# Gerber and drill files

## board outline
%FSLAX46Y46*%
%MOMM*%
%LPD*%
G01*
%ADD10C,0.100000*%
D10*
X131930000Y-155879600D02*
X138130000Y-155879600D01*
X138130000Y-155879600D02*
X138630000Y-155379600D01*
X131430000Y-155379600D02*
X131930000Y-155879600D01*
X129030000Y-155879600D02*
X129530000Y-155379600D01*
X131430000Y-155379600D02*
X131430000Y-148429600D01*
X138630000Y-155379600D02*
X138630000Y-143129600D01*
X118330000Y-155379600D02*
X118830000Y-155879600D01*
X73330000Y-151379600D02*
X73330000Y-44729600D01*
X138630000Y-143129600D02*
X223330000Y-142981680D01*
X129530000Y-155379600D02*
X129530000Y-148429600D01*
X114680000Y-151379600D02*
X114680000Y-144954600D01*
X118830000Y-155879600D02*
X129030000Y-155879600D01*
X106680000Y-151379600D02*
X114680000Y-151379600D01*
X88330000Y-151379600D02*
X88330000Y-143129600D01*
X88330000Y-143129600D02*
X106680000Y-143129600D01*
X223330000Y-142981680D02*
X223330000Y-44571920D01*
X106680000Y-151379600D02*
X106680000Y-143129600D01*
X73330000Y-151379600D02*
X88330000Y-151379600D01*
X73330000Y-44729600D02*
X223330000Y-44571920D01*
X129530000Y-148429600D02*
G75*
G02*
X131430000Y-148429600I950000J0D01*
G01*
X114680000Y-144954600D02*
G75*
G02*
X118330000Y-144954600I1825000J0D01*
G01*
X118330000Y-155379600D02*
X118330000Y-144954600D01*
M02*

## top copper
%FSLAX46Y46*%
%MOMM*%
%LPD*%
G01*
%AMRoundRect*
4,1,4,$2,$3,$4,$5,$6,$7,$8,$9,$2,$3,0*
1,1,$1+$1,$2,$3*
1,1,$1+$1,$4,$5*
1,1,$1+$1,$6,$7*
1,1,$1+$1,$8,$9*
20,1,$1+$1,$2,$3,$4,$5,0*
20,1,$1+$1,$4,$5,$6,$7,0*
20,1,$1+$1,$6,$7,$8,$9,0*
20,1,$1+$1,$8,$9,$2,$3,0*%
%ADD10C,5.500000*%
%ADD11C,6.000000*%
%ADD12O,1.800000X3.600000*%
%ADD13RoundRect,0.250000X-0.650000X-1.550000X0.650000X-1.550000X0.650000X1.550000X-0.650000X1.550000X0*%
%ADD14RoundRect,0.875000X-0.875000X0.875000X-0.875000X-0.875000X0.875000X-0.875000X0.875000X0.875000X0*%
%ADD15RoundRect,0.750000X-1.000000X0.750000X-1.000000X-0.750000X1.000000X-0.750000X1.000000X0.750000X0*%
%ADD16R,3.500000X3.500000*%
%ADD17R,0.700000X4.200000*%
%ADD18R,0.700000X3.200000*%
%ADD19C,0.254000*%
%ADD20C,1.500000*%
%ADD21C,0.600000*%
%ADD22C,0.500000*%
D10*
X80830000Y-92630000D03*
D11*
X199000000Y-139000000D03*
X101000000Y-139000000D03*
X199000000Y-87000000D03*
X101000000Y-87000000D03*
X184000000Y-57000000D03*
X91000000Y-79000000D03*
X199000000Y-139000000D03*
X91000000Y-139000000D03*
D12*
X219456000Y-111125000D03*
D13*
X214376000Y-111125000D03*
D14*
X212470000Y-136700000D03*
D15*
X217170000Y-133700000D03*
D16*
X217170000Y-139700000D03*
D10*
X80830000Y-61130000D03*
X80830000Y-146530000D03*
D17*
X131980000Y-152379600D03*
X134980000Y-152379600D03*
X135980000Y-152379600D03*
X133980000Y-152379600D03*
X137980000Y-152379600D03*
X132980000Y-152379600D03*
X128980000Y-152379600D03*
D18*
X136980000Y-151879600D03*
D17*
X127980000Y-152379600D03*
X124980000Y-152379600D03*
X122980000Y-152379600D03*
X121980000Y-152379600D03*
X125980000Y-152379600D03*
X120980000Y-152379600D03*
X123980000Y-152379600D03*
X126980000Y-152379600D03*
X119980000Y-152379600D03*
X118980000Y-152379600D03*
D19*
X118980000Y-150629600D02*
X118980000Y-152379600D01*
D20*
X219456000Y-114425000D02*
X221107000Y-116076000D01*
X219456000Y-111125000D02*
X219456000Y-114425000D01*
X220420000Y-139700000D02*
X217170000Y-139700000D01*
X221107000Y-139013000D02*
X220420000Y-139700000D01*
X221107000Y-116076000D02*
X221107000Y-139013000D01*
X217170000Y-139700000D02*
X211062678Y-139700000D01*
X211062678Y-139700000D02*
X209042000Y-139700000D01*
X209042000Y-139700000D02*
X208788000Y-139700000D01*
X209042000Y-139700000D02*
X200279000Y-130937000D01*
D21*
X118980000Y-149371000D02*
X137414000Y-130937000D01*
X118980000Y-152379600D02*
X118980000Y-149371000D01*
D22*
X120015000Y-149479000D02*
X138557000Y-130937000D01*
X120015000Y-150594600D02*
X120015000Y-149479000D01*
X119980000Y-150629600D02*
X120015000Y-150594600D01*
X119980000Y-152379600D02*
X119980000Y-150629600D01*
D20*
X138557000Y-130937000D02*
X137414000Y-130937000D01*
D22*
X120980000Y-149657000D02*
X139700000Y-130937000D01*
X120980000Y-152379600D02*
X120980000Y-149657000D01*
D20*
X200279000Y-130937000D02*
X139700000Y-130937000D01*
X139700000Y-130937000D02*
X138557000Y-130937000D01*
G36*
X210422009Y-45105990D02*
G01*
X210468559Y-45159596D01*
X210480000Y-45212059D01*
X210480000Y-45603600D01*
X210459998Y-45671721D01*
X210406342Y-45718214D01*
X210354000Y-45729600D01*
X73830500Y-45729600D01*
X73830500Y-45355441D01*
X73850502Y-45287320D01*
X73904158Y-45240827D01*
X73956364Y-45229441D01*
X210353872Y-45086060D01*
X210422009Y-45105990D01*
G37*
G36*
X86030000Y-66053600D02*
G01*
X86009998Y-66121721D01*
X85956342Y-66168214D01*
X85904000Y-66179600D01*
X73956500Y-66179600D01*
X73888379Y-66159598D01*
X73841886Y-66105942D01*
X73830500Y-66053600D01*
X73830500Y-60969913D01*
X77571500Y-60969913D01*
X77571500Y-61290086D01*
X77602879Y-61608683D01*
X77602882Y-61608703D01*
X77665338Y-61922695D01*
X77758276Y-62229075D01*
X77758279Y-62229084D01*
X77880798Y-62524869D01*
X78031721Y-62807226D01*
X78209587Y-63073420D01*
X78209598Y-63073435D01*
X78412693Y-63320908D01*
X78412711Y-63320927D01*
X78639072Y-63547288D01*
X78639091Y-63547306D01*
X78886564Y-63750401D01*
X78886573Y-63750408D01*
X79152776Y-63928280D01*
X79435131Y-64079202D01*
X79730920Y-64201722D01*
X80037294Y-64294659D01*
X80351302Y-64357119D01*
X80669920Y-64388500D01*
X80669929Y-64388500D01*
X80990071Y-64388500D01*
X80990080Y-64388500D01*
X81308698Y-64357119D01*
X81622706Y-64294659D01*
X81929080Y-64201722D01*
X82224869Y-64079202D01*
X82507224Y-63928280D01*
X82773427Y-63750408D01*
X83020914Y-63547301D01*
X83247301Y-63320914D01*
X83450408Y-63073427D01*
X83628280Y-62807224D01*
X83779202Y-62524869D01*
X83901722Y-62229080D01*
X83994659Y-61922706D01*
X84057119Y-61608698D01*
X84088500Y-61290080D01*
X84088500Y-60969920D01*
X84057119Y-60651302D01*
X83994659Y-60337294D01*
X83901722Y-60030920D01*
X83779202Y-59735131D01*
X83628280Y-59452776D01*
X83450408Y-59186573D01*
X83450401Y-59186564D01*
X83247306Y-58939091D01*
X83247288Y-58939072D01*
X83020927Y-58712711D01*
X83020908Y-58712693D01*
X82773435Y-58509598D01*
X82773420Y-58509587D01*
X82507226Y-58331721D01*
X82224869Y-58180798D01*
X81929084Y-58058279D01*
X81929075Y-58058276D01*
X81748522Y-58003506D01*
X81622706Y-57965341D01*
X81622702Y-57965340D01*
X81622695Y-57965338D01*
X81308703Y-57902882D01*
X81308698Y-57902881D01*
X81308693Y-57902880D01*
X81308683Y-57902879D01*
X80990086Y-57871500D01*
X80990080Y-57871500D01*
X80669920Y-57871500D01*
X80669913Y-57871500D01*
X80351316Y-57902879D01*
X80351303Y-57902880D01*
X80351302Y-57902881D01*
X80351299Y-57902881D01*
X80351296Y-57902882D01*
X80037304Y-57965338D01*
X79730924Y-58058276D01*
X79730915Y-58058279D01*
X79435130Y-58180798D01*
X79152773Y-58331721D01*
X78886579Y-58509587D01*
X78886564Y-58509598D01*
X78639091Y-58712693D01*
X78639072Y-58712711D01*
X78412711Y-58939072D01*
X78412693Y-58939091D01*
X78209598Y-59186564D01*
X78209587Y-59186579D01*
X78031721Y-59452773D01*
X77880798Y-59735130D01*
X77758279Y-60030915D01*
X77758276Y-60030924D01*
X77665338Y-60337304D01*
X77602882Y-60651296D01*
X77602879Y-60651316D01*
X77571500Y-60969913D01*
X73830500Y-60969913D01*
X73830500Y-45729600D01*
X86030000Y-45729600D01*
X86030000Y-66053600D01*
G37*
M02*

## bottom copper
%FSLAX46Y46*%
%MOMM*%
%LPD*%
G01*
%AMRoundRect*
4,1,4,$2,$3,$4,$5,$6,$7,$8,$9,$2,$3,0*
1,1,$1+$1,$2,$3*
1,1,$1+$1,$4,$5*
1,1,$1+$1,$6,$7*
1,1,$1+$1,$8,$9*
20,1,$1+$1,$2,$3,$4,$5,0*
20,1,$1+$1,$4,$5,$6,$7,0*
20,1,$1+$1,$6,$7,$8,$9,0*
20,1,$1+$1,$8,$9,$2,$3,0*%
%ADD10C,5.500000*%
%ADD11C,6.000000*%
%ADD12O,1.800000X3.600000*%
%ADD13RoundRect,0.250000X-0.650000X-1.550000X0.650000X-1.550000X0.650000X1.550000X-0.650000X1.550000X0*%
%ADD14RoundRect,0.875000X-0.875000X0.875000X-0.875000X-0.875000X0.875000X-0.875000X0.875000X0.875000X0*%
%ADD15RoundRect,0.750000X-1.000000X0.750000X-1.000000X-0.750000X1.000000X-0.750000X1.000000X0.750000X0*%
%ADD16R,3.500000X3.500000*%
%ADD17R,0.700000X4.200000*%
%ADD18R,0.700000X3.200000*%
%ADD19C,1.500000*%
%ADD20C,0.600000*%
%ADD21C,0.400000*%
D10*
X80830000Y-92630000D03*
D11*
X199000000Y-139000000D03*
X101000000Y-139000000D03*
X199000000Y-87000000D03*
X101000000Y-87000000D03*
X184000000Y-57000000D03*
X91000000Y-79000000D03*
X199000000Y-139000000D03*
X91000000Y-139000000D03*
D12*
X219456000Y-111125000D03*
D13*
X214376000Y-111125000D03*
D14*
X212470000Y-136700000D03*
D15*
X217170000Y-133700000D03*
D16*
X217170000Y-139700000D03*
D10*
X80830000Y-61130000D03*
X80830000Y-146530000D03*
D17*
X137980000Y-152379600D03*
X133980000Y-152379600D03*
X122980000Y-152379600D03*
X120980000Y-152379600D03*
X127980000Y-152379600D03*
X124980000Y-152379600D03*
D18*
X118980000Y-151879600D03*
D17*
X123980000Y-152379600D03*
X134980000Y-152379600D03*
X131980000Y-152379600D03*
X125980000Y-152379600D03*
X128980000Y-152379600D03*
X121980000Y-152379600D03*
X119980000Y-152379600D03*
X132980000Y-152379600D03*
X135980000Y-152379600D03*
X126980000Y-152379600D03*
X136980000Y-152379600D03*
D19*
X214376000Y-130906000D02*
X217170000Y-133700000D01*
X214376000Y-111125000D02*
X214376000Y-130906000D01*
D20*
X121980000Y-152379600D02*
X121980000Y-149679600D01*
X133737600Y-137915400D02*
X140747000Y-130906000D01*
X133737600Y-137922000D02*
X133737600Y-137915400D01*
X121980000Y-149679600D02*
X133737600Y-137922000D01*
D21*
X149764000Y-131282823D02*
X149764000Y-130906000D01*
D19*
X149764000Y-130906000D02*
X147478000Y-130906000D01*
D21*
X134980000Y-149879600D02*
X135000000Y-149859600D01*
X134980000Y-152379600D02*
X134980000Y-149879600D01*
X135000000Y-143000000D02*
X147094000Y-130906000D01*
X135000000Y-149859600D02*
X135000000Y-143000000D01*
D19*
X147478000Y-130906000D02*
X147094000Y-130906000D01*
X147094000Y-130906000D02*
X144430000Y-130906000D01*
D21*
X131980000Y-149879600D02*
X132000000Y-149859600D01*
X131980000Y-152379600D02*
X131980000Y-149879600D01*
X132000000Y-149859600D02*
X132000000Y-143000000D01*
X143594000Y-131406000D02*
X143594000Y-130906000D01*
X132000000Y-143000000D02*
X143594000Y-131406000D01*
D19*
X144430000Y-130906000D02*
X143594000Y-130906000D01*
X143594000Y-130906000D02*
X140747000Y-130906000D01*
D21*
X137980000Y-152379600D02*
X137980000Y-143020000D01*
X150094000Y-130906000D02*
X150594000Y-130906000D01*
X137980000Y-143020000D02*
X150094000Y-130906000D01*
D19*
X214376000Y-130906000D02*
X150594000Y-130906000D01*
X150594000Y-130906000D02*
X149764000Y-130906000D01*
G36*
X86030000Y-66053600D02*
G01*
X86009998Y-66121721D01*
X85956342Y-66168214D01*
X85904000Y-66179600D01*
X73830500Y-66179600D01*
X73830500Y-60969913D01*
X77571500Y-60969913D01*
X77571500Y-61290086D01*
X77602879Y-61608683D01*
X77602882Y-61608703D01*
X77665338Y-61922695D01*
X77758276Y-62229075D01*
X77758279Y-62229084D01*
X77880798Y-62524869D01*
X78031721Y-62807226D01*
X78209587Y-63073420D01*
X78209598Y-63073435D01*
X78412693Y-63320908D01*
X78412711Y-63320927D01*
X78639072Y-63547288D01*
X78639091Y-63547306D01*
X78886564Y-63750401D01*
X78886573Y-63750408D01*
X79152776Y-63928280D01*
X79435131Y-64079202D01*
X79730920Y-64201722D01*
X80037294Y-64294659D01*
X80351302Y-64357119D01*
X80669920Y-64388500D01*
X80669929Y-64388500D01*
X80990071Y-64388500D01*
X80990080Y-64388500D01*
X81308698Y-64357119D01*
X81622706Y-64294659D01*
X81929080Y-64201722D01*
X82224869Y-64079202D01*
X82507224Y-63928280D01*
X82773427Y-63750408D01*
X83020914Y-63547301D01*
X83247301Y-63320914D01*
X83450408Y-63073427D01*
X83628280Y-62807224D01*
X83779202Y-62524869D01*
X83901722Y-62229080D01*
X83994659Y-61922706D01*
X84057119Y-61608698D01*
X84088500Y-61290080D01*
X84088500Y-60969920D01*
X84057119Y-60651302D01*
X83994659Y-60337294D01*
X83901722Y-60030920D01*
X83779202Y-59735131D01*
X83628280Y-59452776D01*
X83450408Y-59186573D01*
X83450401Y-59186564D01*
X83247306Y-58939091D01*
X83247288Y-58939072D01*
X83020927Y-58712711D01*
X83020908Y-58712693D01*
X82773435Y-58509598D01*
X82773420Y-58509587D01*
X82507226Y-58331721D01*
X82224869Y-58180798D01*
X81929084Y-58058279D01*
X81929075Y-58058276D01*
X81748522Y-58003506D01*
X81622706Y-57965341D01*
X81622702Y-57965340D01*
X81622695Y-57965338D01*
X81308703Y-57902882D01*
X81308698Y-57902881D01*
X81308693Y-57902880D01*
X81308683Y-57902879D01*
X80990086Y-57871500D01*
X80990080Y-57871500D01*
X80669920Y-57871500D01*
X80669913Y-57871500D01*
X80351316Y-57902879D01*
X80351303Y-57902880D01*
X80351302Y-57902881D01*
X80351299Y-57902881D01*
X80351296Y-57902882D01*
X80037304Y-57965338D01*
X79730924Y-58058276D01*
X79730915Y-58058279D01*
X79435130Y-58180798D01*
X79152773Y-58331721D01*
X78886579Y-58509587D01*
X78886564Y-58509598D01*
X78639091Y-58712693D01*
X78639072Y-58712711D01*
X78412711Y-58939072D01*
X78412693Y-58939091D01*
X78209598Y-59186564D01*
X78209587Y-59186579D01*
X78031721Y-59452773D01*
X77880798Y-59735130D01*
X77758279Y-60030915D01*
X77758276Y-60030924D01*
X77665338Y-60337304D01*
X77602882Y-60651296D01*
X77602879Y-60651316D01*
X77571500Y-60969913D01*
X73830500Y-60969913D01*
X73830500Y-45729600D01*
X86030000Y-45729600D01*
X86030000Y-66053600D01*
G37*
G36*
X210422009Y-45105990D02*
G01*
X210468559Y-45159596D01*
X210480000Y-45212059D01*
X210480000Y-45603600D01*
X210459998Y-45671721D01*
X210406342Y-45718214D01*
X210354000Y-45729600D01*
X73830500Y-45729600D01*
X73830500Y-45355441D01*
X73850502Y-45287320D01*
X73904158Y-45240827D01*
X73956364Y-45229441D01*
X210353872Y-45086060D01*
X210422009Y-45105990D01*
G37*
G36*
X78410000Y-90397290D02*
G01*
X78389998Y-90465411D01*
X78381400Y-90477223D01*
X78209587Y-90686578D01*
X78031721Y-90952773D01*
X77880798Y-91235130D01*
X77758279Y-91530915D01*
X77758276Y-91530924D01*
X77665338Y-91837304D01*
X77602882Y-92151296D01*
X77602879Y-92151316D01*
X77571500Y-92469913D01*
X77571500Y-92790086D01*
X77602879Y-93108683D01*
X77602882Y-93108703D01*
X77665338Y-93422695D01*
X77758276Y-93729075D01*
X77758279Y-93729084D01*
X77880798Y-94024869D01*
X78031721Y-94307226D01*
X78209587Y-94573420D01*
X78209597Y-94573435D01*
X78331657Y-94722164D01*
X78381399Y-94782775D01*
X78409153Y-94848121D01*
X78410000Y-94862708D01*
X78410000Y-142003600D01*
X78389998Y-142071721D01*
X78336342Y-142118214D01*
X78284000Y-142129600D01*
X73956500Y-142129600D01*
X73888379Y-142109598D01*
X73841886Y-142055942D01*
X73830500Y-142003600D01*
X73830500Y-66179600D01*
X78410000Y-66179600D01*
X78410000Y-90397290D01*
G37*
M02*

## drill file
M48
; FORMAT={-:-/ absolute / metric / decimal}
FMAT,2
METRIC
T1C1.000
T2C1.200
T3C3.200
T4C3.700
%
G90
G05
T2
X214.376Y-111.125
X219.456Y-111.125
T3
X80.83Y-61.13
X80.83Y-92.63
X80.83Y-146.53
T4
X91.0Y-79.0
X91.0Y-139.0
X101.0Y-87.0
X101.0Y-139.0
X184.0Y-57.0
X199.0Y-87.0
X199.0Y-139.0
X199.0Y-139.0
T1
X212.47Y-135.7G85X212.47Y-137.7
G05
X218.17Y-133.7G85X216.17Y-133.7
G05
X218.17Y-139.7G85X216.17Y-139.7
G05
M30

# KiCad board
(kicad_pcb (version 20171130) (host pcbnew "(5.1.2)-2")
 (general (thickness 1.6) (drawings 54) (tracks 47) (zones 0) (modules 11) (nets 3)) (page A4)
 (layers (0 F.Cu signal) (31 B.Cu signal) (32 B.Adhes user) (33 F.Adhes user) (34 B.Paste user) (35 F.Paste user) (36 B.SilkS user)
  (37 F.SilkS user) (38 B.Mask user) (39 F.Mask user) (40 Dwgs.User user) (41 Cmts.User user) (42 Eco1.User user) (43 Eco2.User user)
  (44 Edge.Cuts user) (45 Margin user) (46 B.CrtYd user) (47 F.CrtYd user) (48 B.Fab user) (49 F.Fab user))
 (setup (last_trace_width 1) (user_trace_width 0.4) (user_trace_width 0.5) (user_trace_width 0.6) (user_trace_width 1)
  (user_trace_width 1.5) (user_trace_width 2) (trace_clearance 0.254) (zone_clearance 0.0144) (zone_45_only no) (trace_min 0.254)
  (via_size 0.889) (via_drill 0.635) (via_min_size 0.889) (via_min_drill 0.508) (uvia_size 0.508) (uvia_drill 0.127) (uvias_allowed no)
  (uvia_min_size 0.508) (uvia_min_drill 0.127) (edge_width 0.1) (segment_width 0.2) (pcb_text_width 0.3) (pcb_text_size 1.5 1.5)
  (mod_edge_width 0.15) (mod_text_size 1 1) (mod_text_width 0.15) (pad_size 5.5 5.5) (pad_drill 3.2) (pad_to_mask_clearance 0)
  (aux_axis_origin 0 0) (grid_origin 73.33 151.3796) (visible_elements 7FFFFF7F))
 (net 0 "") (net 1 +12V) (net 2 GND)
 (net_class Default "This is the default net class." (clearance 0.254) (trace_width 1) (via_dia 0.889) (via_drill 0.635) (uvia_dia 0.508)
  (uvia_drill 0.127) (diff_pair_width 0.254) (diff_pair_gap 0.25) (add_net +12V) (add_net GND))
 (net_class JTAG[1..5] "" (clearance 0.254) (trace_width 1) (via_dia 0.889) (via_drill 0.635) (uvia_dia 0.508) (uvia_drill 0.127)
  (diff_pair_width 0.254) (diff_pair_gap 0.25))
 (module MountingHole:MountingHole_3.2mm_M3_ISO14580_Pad (layer F.Cu) (at 80.83 92.63)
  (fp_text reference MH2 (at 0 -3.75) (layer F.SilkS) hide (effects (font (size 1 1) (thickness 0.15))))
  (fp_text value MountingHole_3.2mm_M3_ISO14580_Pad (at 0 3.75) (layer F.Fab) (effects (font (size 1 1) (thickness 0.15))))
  (pad 1 thru_hole circle (at 0 0) (size 5.5 5.5) (drill 3.2) (layers *.Cu *.Mask)))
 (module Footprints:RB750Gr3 (layer F.Cu) (at 150 113)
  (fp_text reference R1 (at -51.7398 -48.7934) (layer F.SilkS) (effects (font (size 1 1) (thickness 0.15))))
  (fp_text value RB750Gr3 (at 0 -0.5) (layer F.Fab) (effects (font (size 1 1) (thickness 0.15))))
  (pad 4 thru_hole circle (at 49 26) (size 6 6) (drill 3.7) (layers *.Cu *.Mask))
  (pad 3 thru_hole circle (at -49 26) (size 6 6) (drill 3.7) (layers *.Cu *.Mask))
  (pad 2 thru_hole circle (at 49 -26) (size 6 6) (drill 3.7) (layers *.Cu *.Mask))
  (pad 1 thru_hole circle (at -49 -26) (size 6 6) (drill 3.7) (layers *.Cu *.Mask)))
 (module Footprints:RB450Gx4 (layer F.Cu) (at 87 53)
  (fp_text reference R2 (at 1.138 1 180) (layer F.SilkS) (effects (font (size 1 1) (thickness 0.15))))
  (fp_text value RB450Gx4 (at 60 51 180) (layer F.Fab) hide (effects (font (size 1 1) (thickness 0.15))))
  (pad 2 thru_hole circle (at 97 4 180) (size 6 6) (drill 3.7) (layers *.Cu *.Mask))
  (pad 1 thru_hole circle (at 4 26 180) (size 6 6) (drill 3.7) (layers *.Cu *.Mask))
  (pad 4 thru_hole circle (at 112 86 180) (size 6 6) (drill 3.7) (layers *.Cu *.Mask))
  (pad 3 thru_hole circle (at 4 86 180) (size 6 6) (drill 3.7) (layers *.Cu *.Mask)))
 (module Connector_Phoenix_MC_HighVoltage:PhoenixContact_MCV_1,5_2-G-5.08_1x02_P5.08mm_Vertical (layer F.Cu) (at 214.376 111.125)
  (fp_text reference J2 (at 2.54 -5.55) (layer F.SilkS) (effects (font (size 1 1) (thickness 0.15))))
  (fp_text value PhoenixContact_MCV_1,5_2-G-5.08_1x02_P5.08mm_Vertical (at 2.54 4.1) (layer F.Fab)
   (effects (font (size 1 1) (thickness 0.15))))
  (pad 2 thru_hole oval (at 5.08 0) (size 1.8 3.6) (drill 1.2) (layers *.Cu *.Mask) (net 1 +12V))
  (pad 1 thru_hole roundrect (at 0 0) (size 1.8 3.6) (drill 1.2) (layers *.Cu *.Mask) (roundrect_rratio 0.138889) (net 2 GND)))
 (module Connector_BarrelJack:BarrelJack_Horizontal (layer F.Cu) (at 217.17 139.7 270)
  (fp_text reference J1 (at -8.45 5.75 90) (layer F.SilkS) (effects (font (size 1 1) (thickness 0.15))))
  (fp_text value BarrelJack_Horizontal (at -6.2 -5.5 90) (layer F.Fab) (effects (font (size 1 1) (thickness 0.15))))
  (pad 3 thru_hole roundrect (at -3 4.7 270) (size 3.5 3.5) (drill oval 3 1) (layers *.Cu *.Mask) (roundrect_rratio 0.25))
  (pad 2 thru_hole roundrect (at -6 0 270) (size 3 3.5) (drill oval 1 3) (layers *.Cu *.Mask) (roundrect_rratio 0.25) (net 2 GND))
  (pad 1 thru_hole rect (at 0 0 270) (size 3.5 3.5) (drill oval 1 3) (layers *.Cu *.Mask) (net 1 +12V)))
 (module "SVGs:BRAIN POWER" (layer B.Cu) (at 155.575 97.79 180)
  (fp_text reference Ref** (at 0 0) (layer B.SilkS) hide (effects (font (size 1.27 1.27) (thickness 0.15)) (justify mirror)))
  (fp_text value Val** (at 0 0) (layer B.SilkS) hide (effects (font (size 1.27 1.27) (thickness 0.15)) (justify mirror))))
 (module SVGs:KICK (layer F.Cu) (at 148.9456 53.4416)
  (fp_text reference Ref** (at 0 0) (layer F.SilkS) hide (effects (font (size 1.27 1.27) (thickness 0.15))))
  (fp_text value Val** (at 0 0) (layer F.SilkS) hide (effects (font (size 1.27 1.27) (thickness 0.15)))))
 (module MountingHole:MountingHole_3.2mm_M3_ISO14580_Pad (layer F.Cu) (at 80.83 61.13)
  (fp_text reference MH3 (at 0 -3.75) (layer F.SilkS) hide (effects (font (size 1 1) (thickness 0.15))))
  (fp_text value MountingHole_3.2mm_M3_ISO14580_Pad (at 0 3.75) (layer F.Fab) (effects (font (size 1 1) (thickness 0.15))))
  (pad 2 thru_hole circle (at 0 0) (size 5.5 5.5) (drill 3.2) (layers *.Cu *.Mask)))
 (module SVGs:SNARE (layer B.Cu) (at 148.1582 53.5178 180)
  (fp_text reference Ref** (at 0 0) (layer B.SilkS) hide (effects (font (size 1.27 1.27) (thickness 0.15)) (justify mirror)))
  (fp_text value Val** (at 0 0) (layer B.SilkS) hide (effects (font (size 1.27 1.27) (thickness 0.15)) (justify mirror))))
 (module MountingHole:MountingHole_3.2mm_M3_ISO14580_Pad (layer F.Cu) (at 80.83 146.53)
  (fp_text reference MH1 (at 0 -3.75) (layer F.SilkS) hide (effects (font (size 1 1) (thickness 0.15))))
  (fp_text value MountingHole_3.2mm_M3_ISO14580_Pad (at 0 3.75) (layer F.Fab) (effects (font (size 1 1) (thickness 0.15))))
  (pad 1 thru_hole circle (at 0 0) (size 5.5 5.5) (drill 3.2) (layers *.Cu *.Mask)))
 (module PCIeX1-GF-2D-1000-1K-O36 (layer F.Cu) (at 128.48 152.3796)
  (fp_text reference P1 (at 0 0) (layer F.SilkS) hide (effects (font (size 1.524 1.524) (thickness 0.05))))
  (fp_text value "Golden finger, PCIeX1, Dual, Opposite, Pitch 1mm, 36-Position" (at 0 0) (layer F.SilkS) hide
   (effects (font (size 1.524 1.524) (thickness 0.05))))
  (pad B12 smd rect (at 3.5 0) (size 0.7 4.2) (layers F.Cu F.Paste F.Mask))
  (pad B15 smd rect (at 6.5 0) (size 0.7 4.2) (layers F.Cu F.Paste F.Mask))
  (pad B16 smd rect (at 7.5 0) (size 0.7 4.2) (layers F.Cu F.Paste F.Mask))
  (pad B14 smd rect (at 5.5 0) (size 0.7 4.2) (layers F.Cu F.Paste F.Mask))
  (pad B18 smd rect (at 9.5 0) (size 0.7 4.2) (layers F.Cu F.Paste F.Mask))
  (pad B13 smd rect (at 4.5 0) (size 0.7 4.2) (layers F.Cu F.Paste F.Mask))
  (pad B11 smd rect (at 0.5 0) (size 0.7 4.2) (layers F.Cu F.Paste F.Mask))
  (pad B17 smd rect (at 8.5 -0.5) (size 0.7 3.2) (layers F.Cu F.Paste F.Mask))
  (pad B10 smd rect (at -0.5 0) (size 0.7 4.2) (layers F.Cu F.Paste F.Mask))
  (pad B7 smd rect (at -3.5 0) (size 0.7 4.2) (layers F.Cu F.Paste F.Mask))
  (pad B5 smd rect (at -5.5 0) (size 0.7 4.2) (layers F.Cu F.Paste F.Mask))
  (pad B4 smd rect (at -6.5 0) (size 0.7 4.2) (layers F.Cu F.Paste F.Mask))
  (pad B8 smd rect (at -2.5 0) (size 0.7 4.2) (layers F.Cu F.Paste F.Mask))
  (pad B3 smd rect (at -7.5 0) (size 0.7 4.2) (layers F.Cu F.Paste F.Mask) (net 1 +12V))
  (pad B6 smd rect (at -4.5 0) (size 0.7 4.2) (layers F.Cu F.Paste F.Mask))
  (pad B9 smd rect (at -1.5 0) (size 0.7 4.2) (layers F.Cu F.Paste F.Mask))
  (pad B2 smd rect (at -8.5 0) (size 0.7 4.2) (layers F.Cu F.Paste F.Mask) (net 1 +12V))
  (pad B1 smd rect (at -9.5 0) (size 0.7 4.2) (layers F.Cu F.Paste F.Mask) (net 1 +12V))
  (pad A18 smd rect (at 9.5 0) (size 0.7 4.2) (layers B.Cu B.Paste B.Mask) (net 2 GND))
  (pad A14 smd rect (at 5.5 0) (size 0.7 4.2) (layers B.Cu B.Paste B.Mask))
  (pad A5 smd rect (at -5.5 0) (size 0.7 4.2) (layers B.Cu B.Paste B.Mask))
  (pad A3 smd rect (at -7.5 0) (size 0.7 4.2) (layers B.Cu B.Paste B.Mask))
  (pad A10 smd rect (at -0.5 0) (size 0.7 4.2) (layers B.Cu B.Paste B.Mask))
  (pad A7 smd rect (at -3.5 0) (size 0.7 4.2) (layers B.Cu B.Paste B.Mask))
  (pad A1 smd rect (at -9.5 -0.5) (size 0.7 3.2) (layers B.Cu B.Paste B.Mask))
  (pad A6 smd rect (at -4.5 0) (size 0.7 4.2) (layers B.Cu B.Paste B.Mask))
  (pad A15 smd rect (at 6.5 0) (size 0.7 4.2) (layers B.Cu B.Paste B.Mask) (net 2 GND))
  (pad A12 smd rect (at 3.5 0) (size 0.7 4.2) (layers B.Cu B.Paste B.Mask) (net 2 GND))
  (pad A8 smd rect (at -2.5 0) (size 0.7 4.2) (layers B.Cu B.Paste B.Mask))
  (pad A11 smd rect (at 0.5 0) (size 0.7 4.2) (layers B.Cu B.Paste B.Mask))
  (pad A4 smd rect (at -6.5 0) (size 0.7 4.2) (layers B.Cu B.Paste B.Mask) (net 2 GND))
  (pad A2 smd rect (at -8.5 0) (size 0.7 4.2) (layers B.Cu B.Paste B.Mask))
  (pad A13 smd rect (at 4.5 0) (size 0.7 4.2) (layers B.Cu B.Paste B.Mask))
  (pad A16 smd rect (at 7.5 0) (size 0.7 4.2) (layers B.Cu B.Paste B.Mask))
  (pad A9 smd rect (at -1.5 0) (size 0.7 4.2) (layers B.Cu B.Paste B.Mask))
  (pad A17 smd rect (at 8.5 0) (size 0.7 4.2) (layers B.Cu B.Paste B.Mask)))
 (gr_line (start 131.93 155.8796) (end 138.13 155.8796) (layer Edge.Cuts) (width 0.1))
 (gr_line (start 138.13 155.8796) (end 138.63 155.3796) (layer Edge.Cuts) (width 0.1))
 (gr_line (start 131.43 155.3796) (end 131.93 155.8796) (layer Edge.Cuts) (width 0.1))
 (gr_line (start 129.03 155.8796) (end 129.53 155.3796) (layer Edge.Cuts) (width 0.1))
 (gr_line (start 131.43 155.3796) (end 131.43 148.4296) (layer Edge.Cuts) (width 0.1))
 (gr_line (start 138.63 155.3796) (end 138.63 143.1296) (layer Edge.Cuts) (width 0.1))
 (gr_line (start 118.33 155.3796) (end 118.83 155.8796) (layer Edge.Cuts) (width 0.1))
 (gr_line (start 73.33 151.3796) (end 73.33 44.7296) (layer Edge.Cuts) (width 0.1))
 (gr_line (start 138.63 143.1296) (end 223.33 142.98168) (layer Edge.Cuts) (width 0.1))
 (gr_line (start 129.53 155.3796) (end 129.53 148.4296) (layer Edge.Cuts) (width 0.1))
 (gr_line (start 114.68 151.3796) (end 114.68 144.9546) (layer Edge.Cuts) (width 0.1))
 (gr_line (start 118.83 155.8796) (end 129.03 155.8796) (layer Edge.Cuts) (width 0.1))
 (gr_line (start 106.68 151.3796) (end 114.68 151.3796) (layer Edge.Cuts) (width 0.1))
 (gr_line (start 88.33 151.3796) (end 88.33 143.1296) (layer Edge.Cuts) (width 0.1))
 (gr_line (start 88.33 143.1296) (end 106.68 143.1296) (layer Edge.Cuts) (width 0.1))
 (gr_line (start 223.33 142.98168) (end 223.33 44.57192) (layer Edge.Cuts) (width 0.1))
 (gr_line (start 106.68 151.3796) (end 106.68 143.1296) (layer Edge.Cuts) (width 0.1))
 (gr_line (start 73.33 151.3796) (end 88.33 151.3796) (layer Edge.Cuts) (width 0.1))
 (gr_line (start 73.33 44.7296) (end 223.33 44.57192) (layer Edge.Cuts) (width 0.1))
 (gr_arc (start 130.48 148.4296) (end 131.43 148.4296) (angle -180) (layer Edge.Cuts) (width 0.1))
 (gr_arc (start 116.505 144.9546) (end 118.33 144.9546) (angle -180) (layer Edge.Cuts) (width 0.1))
 (gr_line (start 118.33 155.3796) (end 118.33 144.9546) (layer Edge.Cuts) (width 0.1))
 (segment (start 214.376 130.906) (end 217.17 133.7) (width 1.5) (layer B.Cu) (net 2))
 (segment (start 214.376 111.125) (end 214.376 130.906) (width 1.5) (layer B.Cu) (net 2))
 (segment (start 121.98 152.3796) (end 121.98 149.6796) (width 0.6) (layer B.Cu) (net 2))
 (segment (start 133.7376 137.9154) (end 140.747 130.906) (width 0.6) (layer B.Cu) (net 2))
 (segment (start 133.7376 137.922) (end 133.7376 137.9154) (width 0.6) (layer B.Cu) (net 2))
 (segment (start 121.98 149.6796) (end 133.7376 137.922) (width 0.6) (layer B.Cu) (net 2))
 (segment (start 149.764 131.282823) (end 149.764 130.906) (width 0.4) (layer B.Cu) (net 2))
 (segment (start 149.764 130.906) (end 147.478 130.906) (width 1.5) (layer B.Cu) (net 2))
 (segment (start 134.98 149.8796) (end 135 149.8596) (width 0.4) (layer B.Cu) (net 2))
 (segment (start 134.98 152.3796) (end 134.98 149.8796) (width 0.4) (layer B.Cu) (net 2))
 (segment (start 135 143) (end 147.094 130.906) (width 0.4) (layer B.Cu) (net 2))
 (segment (start 135 149.8596) (end 135 143) (width 0.4) (layer B.Cu) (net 2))
 (segment (start 147.478 130.906) (end 147.094 130.906) (width 1.5) (layer B.Cu) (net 2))
 (segment (start 147.094 130.906) (end 144.43 130.906) (width 1.5) (layer B.Cu) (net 2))
 (segment (start 131.98 149.8796) (end 132 149.8596) (width 0.4) (layer B.Cu) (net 2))
 (segment (start 131.98 152.3796) (end 131.98 149.8796) (width 0.4) (layer B.Cu) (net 2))
 (segment (start 132 149.8596) (end 132 143) (width 0.4) (layer B.Cu) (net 2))
 (segment (start 143.594 131.406) (end 143.594 130.906) (width 0.4) (layer B.Cu) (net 2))
 (segment (start 132 143) (end 143.594 131.406) (width 0.4) (layer B.Cu) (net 2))
 (segment (start 144.43 130.906) (end 143.594 130.906) (width 1.5) (layer B.Cu) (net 2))
 (segment (start 143.594 130.906) (end 140.747 130.906) (width 1.5) (layer B.Cu) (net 2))
 (segment (start 137.98 152.3796) (end 137.98 143.02) (width 0.4) (layer B.Cu) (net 2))
 (segment (start 150.094 130.906) (end 150.594 130.906) (width 0.4) (layer B.Cu) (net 2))
 (segment (start 137.98 143.02) (end 150.094 130.906) (width 0.4) (layer B.Cu) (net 2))
 (segment (start 214.376 130.906) (end 150.594 130.906) (width 1.5) (layer B.Cu) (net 2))
 (segment (start 150.594 130.906) (end 149.764 130.906) (width 1.5) (layer B.Cu) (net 2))
 (segment (start 118.98 150.6296) (end 118.98 152.3796) (width 0.254) (layer F.Cu) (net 1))
 (segment (start 219.456 114.425) (end 221.107 116.076) (width 1.5) (layer F.Cu) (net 1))
 (segment (start 219.456 111.125) (end 219.456 114.425) (width 1.5) (layer F.Cu) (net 1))
 (segment (start 220.42 139.7) (end 217.17 139.7) (width 1.5) (layer F.Cu) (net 1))
 (segment (start 221.107 139.013) (end 220.42 139.7) (width 1.5) (layer F.Cu) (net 1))
 (segment (start 221.107 116.076) (end 221.107 139.013) (width 1.5) (layer F.Cu) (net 1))
 (segment (start 217.17 139.7) (end 211.062678 139.7) (width 1.5) (layer F.Cu) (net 1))
 (segment (start 211.062678 139.7) (end 209.042 139.7) (width 1.5) (layer F.Cu) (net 1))
 (segment (start 209.042 139.7) (end 208.788 139.7) (width 1.5) (layer F.Cu) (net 1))
 (segment (start 209.042 139.7) (end 200.279 130.937) (width 1.5) (layer F.Cu) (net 1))
 (segment (start 118.98 149.371) (end 137.414 130.937) (width 0.6) (layer F.Cu) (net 1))
 (segment (start 118.98 152.3796) (end 118.98 149.371) (width 0.6) (layer F.Cu) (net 1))
 (segment (start 120.015 149.479) (end 138.557 130.937) (width 0.5) (layer F.Cu) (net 1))
 (segment (start 120.015 150.5946) (end 120.015 149.479) (width 0.5) (layer F.Cu) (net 1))
 (segment (start 119.98 150.6296) (end 120.015 150.5946) (width 0.5) (layer F.Cu) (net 1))
 (segment (start 119.98 152.3796) (end 119.98 150.6296) (width 0.5) (layer F.Cu) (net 1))
 (segment (start 138.557 130.937) (end 137.414 130.937) (width 1.5) (layer F.Cu) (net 1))
 (segment (start 120.98 149.657) (end 139.7 130.937) (width 0.5) (layer F.Cu) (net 1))
 (segment (start 120.98 152.3796) (end 120.98 149.657) (width 0.5) (layer F.Cu) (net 1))
 (segment (start 200.279 130.937) (end 139.7 130.937) (width 1.5) (layer F.Cu) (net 1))
 (segment (start 139.7 130.937) (end 138.557 130.937) (width 1.5) (layer F.Cu) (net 1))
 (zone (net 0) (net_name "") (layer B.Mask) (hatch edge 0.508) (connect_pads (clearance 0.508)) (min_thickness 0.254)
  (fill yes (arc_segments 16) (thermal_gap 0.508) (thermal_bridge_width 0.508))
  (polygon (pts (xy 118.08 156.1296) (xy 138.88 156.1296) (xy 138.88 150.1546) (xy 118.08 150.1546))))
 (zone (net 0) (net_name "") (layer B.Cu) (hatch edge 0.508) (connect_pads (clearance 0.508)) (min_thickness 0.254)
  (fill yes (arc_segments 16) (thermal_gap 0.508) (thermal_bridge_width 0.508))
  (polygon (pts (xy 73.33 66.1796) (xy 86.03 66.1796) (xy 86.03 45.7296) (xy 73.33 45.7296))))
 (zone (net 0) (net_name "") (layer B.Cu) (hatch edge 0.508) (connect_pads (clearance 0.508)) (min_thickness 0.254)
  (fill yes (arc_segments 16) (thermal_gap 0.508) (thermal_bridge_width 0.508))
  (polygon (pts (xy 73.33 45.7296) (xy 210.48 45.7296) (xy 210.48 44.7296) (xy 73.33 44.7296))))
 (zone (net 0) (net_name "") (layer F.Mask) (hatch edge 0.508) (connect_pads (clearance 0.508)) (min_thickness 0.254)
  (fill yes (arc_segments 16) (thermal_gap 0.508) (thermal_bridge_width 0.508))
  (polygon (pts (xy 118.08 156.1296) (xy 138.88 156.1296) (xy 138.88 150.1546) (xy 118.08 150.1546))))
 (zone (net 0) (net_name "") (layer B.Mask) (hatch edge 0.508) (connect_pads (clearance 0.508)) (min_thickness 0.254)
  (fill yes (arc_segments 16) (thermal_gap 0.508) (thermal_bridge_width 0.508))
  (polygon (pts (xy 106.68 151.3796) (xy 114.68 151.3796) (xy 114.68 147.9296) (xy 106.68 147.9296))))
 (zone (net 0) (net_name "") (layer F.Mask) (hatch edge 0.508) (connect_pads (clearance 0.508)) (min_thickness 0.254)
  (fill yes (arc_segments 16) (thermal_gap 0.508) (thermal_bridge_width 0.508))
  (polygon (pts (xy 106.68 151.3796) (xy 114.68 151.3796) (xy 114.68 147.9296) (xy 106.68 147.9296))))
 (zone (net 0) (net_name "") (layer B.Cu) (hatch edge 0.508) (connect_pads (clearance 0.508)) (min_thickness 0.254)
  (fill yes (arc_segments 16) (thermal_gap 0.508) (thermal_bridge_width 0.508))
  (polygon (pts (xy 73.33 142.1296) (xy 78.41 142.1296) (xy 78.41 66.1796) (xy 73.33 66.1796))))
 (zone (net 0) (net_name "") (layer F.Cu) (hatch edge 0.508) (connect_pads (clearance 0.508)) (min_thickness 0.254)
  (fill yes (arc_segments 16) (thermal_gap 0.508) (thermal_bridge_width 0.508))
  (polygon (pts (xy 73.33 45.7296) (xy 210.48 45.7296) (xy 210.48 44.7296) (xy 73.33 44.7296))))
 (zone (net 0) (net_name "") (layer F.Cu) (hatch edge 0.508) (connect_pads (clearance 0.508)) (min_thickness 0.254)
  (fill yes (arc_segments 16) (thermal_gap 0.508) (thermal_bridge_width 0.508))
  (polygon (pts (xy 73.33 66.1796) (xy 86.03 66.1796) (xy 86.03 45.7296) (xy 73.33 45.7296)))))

